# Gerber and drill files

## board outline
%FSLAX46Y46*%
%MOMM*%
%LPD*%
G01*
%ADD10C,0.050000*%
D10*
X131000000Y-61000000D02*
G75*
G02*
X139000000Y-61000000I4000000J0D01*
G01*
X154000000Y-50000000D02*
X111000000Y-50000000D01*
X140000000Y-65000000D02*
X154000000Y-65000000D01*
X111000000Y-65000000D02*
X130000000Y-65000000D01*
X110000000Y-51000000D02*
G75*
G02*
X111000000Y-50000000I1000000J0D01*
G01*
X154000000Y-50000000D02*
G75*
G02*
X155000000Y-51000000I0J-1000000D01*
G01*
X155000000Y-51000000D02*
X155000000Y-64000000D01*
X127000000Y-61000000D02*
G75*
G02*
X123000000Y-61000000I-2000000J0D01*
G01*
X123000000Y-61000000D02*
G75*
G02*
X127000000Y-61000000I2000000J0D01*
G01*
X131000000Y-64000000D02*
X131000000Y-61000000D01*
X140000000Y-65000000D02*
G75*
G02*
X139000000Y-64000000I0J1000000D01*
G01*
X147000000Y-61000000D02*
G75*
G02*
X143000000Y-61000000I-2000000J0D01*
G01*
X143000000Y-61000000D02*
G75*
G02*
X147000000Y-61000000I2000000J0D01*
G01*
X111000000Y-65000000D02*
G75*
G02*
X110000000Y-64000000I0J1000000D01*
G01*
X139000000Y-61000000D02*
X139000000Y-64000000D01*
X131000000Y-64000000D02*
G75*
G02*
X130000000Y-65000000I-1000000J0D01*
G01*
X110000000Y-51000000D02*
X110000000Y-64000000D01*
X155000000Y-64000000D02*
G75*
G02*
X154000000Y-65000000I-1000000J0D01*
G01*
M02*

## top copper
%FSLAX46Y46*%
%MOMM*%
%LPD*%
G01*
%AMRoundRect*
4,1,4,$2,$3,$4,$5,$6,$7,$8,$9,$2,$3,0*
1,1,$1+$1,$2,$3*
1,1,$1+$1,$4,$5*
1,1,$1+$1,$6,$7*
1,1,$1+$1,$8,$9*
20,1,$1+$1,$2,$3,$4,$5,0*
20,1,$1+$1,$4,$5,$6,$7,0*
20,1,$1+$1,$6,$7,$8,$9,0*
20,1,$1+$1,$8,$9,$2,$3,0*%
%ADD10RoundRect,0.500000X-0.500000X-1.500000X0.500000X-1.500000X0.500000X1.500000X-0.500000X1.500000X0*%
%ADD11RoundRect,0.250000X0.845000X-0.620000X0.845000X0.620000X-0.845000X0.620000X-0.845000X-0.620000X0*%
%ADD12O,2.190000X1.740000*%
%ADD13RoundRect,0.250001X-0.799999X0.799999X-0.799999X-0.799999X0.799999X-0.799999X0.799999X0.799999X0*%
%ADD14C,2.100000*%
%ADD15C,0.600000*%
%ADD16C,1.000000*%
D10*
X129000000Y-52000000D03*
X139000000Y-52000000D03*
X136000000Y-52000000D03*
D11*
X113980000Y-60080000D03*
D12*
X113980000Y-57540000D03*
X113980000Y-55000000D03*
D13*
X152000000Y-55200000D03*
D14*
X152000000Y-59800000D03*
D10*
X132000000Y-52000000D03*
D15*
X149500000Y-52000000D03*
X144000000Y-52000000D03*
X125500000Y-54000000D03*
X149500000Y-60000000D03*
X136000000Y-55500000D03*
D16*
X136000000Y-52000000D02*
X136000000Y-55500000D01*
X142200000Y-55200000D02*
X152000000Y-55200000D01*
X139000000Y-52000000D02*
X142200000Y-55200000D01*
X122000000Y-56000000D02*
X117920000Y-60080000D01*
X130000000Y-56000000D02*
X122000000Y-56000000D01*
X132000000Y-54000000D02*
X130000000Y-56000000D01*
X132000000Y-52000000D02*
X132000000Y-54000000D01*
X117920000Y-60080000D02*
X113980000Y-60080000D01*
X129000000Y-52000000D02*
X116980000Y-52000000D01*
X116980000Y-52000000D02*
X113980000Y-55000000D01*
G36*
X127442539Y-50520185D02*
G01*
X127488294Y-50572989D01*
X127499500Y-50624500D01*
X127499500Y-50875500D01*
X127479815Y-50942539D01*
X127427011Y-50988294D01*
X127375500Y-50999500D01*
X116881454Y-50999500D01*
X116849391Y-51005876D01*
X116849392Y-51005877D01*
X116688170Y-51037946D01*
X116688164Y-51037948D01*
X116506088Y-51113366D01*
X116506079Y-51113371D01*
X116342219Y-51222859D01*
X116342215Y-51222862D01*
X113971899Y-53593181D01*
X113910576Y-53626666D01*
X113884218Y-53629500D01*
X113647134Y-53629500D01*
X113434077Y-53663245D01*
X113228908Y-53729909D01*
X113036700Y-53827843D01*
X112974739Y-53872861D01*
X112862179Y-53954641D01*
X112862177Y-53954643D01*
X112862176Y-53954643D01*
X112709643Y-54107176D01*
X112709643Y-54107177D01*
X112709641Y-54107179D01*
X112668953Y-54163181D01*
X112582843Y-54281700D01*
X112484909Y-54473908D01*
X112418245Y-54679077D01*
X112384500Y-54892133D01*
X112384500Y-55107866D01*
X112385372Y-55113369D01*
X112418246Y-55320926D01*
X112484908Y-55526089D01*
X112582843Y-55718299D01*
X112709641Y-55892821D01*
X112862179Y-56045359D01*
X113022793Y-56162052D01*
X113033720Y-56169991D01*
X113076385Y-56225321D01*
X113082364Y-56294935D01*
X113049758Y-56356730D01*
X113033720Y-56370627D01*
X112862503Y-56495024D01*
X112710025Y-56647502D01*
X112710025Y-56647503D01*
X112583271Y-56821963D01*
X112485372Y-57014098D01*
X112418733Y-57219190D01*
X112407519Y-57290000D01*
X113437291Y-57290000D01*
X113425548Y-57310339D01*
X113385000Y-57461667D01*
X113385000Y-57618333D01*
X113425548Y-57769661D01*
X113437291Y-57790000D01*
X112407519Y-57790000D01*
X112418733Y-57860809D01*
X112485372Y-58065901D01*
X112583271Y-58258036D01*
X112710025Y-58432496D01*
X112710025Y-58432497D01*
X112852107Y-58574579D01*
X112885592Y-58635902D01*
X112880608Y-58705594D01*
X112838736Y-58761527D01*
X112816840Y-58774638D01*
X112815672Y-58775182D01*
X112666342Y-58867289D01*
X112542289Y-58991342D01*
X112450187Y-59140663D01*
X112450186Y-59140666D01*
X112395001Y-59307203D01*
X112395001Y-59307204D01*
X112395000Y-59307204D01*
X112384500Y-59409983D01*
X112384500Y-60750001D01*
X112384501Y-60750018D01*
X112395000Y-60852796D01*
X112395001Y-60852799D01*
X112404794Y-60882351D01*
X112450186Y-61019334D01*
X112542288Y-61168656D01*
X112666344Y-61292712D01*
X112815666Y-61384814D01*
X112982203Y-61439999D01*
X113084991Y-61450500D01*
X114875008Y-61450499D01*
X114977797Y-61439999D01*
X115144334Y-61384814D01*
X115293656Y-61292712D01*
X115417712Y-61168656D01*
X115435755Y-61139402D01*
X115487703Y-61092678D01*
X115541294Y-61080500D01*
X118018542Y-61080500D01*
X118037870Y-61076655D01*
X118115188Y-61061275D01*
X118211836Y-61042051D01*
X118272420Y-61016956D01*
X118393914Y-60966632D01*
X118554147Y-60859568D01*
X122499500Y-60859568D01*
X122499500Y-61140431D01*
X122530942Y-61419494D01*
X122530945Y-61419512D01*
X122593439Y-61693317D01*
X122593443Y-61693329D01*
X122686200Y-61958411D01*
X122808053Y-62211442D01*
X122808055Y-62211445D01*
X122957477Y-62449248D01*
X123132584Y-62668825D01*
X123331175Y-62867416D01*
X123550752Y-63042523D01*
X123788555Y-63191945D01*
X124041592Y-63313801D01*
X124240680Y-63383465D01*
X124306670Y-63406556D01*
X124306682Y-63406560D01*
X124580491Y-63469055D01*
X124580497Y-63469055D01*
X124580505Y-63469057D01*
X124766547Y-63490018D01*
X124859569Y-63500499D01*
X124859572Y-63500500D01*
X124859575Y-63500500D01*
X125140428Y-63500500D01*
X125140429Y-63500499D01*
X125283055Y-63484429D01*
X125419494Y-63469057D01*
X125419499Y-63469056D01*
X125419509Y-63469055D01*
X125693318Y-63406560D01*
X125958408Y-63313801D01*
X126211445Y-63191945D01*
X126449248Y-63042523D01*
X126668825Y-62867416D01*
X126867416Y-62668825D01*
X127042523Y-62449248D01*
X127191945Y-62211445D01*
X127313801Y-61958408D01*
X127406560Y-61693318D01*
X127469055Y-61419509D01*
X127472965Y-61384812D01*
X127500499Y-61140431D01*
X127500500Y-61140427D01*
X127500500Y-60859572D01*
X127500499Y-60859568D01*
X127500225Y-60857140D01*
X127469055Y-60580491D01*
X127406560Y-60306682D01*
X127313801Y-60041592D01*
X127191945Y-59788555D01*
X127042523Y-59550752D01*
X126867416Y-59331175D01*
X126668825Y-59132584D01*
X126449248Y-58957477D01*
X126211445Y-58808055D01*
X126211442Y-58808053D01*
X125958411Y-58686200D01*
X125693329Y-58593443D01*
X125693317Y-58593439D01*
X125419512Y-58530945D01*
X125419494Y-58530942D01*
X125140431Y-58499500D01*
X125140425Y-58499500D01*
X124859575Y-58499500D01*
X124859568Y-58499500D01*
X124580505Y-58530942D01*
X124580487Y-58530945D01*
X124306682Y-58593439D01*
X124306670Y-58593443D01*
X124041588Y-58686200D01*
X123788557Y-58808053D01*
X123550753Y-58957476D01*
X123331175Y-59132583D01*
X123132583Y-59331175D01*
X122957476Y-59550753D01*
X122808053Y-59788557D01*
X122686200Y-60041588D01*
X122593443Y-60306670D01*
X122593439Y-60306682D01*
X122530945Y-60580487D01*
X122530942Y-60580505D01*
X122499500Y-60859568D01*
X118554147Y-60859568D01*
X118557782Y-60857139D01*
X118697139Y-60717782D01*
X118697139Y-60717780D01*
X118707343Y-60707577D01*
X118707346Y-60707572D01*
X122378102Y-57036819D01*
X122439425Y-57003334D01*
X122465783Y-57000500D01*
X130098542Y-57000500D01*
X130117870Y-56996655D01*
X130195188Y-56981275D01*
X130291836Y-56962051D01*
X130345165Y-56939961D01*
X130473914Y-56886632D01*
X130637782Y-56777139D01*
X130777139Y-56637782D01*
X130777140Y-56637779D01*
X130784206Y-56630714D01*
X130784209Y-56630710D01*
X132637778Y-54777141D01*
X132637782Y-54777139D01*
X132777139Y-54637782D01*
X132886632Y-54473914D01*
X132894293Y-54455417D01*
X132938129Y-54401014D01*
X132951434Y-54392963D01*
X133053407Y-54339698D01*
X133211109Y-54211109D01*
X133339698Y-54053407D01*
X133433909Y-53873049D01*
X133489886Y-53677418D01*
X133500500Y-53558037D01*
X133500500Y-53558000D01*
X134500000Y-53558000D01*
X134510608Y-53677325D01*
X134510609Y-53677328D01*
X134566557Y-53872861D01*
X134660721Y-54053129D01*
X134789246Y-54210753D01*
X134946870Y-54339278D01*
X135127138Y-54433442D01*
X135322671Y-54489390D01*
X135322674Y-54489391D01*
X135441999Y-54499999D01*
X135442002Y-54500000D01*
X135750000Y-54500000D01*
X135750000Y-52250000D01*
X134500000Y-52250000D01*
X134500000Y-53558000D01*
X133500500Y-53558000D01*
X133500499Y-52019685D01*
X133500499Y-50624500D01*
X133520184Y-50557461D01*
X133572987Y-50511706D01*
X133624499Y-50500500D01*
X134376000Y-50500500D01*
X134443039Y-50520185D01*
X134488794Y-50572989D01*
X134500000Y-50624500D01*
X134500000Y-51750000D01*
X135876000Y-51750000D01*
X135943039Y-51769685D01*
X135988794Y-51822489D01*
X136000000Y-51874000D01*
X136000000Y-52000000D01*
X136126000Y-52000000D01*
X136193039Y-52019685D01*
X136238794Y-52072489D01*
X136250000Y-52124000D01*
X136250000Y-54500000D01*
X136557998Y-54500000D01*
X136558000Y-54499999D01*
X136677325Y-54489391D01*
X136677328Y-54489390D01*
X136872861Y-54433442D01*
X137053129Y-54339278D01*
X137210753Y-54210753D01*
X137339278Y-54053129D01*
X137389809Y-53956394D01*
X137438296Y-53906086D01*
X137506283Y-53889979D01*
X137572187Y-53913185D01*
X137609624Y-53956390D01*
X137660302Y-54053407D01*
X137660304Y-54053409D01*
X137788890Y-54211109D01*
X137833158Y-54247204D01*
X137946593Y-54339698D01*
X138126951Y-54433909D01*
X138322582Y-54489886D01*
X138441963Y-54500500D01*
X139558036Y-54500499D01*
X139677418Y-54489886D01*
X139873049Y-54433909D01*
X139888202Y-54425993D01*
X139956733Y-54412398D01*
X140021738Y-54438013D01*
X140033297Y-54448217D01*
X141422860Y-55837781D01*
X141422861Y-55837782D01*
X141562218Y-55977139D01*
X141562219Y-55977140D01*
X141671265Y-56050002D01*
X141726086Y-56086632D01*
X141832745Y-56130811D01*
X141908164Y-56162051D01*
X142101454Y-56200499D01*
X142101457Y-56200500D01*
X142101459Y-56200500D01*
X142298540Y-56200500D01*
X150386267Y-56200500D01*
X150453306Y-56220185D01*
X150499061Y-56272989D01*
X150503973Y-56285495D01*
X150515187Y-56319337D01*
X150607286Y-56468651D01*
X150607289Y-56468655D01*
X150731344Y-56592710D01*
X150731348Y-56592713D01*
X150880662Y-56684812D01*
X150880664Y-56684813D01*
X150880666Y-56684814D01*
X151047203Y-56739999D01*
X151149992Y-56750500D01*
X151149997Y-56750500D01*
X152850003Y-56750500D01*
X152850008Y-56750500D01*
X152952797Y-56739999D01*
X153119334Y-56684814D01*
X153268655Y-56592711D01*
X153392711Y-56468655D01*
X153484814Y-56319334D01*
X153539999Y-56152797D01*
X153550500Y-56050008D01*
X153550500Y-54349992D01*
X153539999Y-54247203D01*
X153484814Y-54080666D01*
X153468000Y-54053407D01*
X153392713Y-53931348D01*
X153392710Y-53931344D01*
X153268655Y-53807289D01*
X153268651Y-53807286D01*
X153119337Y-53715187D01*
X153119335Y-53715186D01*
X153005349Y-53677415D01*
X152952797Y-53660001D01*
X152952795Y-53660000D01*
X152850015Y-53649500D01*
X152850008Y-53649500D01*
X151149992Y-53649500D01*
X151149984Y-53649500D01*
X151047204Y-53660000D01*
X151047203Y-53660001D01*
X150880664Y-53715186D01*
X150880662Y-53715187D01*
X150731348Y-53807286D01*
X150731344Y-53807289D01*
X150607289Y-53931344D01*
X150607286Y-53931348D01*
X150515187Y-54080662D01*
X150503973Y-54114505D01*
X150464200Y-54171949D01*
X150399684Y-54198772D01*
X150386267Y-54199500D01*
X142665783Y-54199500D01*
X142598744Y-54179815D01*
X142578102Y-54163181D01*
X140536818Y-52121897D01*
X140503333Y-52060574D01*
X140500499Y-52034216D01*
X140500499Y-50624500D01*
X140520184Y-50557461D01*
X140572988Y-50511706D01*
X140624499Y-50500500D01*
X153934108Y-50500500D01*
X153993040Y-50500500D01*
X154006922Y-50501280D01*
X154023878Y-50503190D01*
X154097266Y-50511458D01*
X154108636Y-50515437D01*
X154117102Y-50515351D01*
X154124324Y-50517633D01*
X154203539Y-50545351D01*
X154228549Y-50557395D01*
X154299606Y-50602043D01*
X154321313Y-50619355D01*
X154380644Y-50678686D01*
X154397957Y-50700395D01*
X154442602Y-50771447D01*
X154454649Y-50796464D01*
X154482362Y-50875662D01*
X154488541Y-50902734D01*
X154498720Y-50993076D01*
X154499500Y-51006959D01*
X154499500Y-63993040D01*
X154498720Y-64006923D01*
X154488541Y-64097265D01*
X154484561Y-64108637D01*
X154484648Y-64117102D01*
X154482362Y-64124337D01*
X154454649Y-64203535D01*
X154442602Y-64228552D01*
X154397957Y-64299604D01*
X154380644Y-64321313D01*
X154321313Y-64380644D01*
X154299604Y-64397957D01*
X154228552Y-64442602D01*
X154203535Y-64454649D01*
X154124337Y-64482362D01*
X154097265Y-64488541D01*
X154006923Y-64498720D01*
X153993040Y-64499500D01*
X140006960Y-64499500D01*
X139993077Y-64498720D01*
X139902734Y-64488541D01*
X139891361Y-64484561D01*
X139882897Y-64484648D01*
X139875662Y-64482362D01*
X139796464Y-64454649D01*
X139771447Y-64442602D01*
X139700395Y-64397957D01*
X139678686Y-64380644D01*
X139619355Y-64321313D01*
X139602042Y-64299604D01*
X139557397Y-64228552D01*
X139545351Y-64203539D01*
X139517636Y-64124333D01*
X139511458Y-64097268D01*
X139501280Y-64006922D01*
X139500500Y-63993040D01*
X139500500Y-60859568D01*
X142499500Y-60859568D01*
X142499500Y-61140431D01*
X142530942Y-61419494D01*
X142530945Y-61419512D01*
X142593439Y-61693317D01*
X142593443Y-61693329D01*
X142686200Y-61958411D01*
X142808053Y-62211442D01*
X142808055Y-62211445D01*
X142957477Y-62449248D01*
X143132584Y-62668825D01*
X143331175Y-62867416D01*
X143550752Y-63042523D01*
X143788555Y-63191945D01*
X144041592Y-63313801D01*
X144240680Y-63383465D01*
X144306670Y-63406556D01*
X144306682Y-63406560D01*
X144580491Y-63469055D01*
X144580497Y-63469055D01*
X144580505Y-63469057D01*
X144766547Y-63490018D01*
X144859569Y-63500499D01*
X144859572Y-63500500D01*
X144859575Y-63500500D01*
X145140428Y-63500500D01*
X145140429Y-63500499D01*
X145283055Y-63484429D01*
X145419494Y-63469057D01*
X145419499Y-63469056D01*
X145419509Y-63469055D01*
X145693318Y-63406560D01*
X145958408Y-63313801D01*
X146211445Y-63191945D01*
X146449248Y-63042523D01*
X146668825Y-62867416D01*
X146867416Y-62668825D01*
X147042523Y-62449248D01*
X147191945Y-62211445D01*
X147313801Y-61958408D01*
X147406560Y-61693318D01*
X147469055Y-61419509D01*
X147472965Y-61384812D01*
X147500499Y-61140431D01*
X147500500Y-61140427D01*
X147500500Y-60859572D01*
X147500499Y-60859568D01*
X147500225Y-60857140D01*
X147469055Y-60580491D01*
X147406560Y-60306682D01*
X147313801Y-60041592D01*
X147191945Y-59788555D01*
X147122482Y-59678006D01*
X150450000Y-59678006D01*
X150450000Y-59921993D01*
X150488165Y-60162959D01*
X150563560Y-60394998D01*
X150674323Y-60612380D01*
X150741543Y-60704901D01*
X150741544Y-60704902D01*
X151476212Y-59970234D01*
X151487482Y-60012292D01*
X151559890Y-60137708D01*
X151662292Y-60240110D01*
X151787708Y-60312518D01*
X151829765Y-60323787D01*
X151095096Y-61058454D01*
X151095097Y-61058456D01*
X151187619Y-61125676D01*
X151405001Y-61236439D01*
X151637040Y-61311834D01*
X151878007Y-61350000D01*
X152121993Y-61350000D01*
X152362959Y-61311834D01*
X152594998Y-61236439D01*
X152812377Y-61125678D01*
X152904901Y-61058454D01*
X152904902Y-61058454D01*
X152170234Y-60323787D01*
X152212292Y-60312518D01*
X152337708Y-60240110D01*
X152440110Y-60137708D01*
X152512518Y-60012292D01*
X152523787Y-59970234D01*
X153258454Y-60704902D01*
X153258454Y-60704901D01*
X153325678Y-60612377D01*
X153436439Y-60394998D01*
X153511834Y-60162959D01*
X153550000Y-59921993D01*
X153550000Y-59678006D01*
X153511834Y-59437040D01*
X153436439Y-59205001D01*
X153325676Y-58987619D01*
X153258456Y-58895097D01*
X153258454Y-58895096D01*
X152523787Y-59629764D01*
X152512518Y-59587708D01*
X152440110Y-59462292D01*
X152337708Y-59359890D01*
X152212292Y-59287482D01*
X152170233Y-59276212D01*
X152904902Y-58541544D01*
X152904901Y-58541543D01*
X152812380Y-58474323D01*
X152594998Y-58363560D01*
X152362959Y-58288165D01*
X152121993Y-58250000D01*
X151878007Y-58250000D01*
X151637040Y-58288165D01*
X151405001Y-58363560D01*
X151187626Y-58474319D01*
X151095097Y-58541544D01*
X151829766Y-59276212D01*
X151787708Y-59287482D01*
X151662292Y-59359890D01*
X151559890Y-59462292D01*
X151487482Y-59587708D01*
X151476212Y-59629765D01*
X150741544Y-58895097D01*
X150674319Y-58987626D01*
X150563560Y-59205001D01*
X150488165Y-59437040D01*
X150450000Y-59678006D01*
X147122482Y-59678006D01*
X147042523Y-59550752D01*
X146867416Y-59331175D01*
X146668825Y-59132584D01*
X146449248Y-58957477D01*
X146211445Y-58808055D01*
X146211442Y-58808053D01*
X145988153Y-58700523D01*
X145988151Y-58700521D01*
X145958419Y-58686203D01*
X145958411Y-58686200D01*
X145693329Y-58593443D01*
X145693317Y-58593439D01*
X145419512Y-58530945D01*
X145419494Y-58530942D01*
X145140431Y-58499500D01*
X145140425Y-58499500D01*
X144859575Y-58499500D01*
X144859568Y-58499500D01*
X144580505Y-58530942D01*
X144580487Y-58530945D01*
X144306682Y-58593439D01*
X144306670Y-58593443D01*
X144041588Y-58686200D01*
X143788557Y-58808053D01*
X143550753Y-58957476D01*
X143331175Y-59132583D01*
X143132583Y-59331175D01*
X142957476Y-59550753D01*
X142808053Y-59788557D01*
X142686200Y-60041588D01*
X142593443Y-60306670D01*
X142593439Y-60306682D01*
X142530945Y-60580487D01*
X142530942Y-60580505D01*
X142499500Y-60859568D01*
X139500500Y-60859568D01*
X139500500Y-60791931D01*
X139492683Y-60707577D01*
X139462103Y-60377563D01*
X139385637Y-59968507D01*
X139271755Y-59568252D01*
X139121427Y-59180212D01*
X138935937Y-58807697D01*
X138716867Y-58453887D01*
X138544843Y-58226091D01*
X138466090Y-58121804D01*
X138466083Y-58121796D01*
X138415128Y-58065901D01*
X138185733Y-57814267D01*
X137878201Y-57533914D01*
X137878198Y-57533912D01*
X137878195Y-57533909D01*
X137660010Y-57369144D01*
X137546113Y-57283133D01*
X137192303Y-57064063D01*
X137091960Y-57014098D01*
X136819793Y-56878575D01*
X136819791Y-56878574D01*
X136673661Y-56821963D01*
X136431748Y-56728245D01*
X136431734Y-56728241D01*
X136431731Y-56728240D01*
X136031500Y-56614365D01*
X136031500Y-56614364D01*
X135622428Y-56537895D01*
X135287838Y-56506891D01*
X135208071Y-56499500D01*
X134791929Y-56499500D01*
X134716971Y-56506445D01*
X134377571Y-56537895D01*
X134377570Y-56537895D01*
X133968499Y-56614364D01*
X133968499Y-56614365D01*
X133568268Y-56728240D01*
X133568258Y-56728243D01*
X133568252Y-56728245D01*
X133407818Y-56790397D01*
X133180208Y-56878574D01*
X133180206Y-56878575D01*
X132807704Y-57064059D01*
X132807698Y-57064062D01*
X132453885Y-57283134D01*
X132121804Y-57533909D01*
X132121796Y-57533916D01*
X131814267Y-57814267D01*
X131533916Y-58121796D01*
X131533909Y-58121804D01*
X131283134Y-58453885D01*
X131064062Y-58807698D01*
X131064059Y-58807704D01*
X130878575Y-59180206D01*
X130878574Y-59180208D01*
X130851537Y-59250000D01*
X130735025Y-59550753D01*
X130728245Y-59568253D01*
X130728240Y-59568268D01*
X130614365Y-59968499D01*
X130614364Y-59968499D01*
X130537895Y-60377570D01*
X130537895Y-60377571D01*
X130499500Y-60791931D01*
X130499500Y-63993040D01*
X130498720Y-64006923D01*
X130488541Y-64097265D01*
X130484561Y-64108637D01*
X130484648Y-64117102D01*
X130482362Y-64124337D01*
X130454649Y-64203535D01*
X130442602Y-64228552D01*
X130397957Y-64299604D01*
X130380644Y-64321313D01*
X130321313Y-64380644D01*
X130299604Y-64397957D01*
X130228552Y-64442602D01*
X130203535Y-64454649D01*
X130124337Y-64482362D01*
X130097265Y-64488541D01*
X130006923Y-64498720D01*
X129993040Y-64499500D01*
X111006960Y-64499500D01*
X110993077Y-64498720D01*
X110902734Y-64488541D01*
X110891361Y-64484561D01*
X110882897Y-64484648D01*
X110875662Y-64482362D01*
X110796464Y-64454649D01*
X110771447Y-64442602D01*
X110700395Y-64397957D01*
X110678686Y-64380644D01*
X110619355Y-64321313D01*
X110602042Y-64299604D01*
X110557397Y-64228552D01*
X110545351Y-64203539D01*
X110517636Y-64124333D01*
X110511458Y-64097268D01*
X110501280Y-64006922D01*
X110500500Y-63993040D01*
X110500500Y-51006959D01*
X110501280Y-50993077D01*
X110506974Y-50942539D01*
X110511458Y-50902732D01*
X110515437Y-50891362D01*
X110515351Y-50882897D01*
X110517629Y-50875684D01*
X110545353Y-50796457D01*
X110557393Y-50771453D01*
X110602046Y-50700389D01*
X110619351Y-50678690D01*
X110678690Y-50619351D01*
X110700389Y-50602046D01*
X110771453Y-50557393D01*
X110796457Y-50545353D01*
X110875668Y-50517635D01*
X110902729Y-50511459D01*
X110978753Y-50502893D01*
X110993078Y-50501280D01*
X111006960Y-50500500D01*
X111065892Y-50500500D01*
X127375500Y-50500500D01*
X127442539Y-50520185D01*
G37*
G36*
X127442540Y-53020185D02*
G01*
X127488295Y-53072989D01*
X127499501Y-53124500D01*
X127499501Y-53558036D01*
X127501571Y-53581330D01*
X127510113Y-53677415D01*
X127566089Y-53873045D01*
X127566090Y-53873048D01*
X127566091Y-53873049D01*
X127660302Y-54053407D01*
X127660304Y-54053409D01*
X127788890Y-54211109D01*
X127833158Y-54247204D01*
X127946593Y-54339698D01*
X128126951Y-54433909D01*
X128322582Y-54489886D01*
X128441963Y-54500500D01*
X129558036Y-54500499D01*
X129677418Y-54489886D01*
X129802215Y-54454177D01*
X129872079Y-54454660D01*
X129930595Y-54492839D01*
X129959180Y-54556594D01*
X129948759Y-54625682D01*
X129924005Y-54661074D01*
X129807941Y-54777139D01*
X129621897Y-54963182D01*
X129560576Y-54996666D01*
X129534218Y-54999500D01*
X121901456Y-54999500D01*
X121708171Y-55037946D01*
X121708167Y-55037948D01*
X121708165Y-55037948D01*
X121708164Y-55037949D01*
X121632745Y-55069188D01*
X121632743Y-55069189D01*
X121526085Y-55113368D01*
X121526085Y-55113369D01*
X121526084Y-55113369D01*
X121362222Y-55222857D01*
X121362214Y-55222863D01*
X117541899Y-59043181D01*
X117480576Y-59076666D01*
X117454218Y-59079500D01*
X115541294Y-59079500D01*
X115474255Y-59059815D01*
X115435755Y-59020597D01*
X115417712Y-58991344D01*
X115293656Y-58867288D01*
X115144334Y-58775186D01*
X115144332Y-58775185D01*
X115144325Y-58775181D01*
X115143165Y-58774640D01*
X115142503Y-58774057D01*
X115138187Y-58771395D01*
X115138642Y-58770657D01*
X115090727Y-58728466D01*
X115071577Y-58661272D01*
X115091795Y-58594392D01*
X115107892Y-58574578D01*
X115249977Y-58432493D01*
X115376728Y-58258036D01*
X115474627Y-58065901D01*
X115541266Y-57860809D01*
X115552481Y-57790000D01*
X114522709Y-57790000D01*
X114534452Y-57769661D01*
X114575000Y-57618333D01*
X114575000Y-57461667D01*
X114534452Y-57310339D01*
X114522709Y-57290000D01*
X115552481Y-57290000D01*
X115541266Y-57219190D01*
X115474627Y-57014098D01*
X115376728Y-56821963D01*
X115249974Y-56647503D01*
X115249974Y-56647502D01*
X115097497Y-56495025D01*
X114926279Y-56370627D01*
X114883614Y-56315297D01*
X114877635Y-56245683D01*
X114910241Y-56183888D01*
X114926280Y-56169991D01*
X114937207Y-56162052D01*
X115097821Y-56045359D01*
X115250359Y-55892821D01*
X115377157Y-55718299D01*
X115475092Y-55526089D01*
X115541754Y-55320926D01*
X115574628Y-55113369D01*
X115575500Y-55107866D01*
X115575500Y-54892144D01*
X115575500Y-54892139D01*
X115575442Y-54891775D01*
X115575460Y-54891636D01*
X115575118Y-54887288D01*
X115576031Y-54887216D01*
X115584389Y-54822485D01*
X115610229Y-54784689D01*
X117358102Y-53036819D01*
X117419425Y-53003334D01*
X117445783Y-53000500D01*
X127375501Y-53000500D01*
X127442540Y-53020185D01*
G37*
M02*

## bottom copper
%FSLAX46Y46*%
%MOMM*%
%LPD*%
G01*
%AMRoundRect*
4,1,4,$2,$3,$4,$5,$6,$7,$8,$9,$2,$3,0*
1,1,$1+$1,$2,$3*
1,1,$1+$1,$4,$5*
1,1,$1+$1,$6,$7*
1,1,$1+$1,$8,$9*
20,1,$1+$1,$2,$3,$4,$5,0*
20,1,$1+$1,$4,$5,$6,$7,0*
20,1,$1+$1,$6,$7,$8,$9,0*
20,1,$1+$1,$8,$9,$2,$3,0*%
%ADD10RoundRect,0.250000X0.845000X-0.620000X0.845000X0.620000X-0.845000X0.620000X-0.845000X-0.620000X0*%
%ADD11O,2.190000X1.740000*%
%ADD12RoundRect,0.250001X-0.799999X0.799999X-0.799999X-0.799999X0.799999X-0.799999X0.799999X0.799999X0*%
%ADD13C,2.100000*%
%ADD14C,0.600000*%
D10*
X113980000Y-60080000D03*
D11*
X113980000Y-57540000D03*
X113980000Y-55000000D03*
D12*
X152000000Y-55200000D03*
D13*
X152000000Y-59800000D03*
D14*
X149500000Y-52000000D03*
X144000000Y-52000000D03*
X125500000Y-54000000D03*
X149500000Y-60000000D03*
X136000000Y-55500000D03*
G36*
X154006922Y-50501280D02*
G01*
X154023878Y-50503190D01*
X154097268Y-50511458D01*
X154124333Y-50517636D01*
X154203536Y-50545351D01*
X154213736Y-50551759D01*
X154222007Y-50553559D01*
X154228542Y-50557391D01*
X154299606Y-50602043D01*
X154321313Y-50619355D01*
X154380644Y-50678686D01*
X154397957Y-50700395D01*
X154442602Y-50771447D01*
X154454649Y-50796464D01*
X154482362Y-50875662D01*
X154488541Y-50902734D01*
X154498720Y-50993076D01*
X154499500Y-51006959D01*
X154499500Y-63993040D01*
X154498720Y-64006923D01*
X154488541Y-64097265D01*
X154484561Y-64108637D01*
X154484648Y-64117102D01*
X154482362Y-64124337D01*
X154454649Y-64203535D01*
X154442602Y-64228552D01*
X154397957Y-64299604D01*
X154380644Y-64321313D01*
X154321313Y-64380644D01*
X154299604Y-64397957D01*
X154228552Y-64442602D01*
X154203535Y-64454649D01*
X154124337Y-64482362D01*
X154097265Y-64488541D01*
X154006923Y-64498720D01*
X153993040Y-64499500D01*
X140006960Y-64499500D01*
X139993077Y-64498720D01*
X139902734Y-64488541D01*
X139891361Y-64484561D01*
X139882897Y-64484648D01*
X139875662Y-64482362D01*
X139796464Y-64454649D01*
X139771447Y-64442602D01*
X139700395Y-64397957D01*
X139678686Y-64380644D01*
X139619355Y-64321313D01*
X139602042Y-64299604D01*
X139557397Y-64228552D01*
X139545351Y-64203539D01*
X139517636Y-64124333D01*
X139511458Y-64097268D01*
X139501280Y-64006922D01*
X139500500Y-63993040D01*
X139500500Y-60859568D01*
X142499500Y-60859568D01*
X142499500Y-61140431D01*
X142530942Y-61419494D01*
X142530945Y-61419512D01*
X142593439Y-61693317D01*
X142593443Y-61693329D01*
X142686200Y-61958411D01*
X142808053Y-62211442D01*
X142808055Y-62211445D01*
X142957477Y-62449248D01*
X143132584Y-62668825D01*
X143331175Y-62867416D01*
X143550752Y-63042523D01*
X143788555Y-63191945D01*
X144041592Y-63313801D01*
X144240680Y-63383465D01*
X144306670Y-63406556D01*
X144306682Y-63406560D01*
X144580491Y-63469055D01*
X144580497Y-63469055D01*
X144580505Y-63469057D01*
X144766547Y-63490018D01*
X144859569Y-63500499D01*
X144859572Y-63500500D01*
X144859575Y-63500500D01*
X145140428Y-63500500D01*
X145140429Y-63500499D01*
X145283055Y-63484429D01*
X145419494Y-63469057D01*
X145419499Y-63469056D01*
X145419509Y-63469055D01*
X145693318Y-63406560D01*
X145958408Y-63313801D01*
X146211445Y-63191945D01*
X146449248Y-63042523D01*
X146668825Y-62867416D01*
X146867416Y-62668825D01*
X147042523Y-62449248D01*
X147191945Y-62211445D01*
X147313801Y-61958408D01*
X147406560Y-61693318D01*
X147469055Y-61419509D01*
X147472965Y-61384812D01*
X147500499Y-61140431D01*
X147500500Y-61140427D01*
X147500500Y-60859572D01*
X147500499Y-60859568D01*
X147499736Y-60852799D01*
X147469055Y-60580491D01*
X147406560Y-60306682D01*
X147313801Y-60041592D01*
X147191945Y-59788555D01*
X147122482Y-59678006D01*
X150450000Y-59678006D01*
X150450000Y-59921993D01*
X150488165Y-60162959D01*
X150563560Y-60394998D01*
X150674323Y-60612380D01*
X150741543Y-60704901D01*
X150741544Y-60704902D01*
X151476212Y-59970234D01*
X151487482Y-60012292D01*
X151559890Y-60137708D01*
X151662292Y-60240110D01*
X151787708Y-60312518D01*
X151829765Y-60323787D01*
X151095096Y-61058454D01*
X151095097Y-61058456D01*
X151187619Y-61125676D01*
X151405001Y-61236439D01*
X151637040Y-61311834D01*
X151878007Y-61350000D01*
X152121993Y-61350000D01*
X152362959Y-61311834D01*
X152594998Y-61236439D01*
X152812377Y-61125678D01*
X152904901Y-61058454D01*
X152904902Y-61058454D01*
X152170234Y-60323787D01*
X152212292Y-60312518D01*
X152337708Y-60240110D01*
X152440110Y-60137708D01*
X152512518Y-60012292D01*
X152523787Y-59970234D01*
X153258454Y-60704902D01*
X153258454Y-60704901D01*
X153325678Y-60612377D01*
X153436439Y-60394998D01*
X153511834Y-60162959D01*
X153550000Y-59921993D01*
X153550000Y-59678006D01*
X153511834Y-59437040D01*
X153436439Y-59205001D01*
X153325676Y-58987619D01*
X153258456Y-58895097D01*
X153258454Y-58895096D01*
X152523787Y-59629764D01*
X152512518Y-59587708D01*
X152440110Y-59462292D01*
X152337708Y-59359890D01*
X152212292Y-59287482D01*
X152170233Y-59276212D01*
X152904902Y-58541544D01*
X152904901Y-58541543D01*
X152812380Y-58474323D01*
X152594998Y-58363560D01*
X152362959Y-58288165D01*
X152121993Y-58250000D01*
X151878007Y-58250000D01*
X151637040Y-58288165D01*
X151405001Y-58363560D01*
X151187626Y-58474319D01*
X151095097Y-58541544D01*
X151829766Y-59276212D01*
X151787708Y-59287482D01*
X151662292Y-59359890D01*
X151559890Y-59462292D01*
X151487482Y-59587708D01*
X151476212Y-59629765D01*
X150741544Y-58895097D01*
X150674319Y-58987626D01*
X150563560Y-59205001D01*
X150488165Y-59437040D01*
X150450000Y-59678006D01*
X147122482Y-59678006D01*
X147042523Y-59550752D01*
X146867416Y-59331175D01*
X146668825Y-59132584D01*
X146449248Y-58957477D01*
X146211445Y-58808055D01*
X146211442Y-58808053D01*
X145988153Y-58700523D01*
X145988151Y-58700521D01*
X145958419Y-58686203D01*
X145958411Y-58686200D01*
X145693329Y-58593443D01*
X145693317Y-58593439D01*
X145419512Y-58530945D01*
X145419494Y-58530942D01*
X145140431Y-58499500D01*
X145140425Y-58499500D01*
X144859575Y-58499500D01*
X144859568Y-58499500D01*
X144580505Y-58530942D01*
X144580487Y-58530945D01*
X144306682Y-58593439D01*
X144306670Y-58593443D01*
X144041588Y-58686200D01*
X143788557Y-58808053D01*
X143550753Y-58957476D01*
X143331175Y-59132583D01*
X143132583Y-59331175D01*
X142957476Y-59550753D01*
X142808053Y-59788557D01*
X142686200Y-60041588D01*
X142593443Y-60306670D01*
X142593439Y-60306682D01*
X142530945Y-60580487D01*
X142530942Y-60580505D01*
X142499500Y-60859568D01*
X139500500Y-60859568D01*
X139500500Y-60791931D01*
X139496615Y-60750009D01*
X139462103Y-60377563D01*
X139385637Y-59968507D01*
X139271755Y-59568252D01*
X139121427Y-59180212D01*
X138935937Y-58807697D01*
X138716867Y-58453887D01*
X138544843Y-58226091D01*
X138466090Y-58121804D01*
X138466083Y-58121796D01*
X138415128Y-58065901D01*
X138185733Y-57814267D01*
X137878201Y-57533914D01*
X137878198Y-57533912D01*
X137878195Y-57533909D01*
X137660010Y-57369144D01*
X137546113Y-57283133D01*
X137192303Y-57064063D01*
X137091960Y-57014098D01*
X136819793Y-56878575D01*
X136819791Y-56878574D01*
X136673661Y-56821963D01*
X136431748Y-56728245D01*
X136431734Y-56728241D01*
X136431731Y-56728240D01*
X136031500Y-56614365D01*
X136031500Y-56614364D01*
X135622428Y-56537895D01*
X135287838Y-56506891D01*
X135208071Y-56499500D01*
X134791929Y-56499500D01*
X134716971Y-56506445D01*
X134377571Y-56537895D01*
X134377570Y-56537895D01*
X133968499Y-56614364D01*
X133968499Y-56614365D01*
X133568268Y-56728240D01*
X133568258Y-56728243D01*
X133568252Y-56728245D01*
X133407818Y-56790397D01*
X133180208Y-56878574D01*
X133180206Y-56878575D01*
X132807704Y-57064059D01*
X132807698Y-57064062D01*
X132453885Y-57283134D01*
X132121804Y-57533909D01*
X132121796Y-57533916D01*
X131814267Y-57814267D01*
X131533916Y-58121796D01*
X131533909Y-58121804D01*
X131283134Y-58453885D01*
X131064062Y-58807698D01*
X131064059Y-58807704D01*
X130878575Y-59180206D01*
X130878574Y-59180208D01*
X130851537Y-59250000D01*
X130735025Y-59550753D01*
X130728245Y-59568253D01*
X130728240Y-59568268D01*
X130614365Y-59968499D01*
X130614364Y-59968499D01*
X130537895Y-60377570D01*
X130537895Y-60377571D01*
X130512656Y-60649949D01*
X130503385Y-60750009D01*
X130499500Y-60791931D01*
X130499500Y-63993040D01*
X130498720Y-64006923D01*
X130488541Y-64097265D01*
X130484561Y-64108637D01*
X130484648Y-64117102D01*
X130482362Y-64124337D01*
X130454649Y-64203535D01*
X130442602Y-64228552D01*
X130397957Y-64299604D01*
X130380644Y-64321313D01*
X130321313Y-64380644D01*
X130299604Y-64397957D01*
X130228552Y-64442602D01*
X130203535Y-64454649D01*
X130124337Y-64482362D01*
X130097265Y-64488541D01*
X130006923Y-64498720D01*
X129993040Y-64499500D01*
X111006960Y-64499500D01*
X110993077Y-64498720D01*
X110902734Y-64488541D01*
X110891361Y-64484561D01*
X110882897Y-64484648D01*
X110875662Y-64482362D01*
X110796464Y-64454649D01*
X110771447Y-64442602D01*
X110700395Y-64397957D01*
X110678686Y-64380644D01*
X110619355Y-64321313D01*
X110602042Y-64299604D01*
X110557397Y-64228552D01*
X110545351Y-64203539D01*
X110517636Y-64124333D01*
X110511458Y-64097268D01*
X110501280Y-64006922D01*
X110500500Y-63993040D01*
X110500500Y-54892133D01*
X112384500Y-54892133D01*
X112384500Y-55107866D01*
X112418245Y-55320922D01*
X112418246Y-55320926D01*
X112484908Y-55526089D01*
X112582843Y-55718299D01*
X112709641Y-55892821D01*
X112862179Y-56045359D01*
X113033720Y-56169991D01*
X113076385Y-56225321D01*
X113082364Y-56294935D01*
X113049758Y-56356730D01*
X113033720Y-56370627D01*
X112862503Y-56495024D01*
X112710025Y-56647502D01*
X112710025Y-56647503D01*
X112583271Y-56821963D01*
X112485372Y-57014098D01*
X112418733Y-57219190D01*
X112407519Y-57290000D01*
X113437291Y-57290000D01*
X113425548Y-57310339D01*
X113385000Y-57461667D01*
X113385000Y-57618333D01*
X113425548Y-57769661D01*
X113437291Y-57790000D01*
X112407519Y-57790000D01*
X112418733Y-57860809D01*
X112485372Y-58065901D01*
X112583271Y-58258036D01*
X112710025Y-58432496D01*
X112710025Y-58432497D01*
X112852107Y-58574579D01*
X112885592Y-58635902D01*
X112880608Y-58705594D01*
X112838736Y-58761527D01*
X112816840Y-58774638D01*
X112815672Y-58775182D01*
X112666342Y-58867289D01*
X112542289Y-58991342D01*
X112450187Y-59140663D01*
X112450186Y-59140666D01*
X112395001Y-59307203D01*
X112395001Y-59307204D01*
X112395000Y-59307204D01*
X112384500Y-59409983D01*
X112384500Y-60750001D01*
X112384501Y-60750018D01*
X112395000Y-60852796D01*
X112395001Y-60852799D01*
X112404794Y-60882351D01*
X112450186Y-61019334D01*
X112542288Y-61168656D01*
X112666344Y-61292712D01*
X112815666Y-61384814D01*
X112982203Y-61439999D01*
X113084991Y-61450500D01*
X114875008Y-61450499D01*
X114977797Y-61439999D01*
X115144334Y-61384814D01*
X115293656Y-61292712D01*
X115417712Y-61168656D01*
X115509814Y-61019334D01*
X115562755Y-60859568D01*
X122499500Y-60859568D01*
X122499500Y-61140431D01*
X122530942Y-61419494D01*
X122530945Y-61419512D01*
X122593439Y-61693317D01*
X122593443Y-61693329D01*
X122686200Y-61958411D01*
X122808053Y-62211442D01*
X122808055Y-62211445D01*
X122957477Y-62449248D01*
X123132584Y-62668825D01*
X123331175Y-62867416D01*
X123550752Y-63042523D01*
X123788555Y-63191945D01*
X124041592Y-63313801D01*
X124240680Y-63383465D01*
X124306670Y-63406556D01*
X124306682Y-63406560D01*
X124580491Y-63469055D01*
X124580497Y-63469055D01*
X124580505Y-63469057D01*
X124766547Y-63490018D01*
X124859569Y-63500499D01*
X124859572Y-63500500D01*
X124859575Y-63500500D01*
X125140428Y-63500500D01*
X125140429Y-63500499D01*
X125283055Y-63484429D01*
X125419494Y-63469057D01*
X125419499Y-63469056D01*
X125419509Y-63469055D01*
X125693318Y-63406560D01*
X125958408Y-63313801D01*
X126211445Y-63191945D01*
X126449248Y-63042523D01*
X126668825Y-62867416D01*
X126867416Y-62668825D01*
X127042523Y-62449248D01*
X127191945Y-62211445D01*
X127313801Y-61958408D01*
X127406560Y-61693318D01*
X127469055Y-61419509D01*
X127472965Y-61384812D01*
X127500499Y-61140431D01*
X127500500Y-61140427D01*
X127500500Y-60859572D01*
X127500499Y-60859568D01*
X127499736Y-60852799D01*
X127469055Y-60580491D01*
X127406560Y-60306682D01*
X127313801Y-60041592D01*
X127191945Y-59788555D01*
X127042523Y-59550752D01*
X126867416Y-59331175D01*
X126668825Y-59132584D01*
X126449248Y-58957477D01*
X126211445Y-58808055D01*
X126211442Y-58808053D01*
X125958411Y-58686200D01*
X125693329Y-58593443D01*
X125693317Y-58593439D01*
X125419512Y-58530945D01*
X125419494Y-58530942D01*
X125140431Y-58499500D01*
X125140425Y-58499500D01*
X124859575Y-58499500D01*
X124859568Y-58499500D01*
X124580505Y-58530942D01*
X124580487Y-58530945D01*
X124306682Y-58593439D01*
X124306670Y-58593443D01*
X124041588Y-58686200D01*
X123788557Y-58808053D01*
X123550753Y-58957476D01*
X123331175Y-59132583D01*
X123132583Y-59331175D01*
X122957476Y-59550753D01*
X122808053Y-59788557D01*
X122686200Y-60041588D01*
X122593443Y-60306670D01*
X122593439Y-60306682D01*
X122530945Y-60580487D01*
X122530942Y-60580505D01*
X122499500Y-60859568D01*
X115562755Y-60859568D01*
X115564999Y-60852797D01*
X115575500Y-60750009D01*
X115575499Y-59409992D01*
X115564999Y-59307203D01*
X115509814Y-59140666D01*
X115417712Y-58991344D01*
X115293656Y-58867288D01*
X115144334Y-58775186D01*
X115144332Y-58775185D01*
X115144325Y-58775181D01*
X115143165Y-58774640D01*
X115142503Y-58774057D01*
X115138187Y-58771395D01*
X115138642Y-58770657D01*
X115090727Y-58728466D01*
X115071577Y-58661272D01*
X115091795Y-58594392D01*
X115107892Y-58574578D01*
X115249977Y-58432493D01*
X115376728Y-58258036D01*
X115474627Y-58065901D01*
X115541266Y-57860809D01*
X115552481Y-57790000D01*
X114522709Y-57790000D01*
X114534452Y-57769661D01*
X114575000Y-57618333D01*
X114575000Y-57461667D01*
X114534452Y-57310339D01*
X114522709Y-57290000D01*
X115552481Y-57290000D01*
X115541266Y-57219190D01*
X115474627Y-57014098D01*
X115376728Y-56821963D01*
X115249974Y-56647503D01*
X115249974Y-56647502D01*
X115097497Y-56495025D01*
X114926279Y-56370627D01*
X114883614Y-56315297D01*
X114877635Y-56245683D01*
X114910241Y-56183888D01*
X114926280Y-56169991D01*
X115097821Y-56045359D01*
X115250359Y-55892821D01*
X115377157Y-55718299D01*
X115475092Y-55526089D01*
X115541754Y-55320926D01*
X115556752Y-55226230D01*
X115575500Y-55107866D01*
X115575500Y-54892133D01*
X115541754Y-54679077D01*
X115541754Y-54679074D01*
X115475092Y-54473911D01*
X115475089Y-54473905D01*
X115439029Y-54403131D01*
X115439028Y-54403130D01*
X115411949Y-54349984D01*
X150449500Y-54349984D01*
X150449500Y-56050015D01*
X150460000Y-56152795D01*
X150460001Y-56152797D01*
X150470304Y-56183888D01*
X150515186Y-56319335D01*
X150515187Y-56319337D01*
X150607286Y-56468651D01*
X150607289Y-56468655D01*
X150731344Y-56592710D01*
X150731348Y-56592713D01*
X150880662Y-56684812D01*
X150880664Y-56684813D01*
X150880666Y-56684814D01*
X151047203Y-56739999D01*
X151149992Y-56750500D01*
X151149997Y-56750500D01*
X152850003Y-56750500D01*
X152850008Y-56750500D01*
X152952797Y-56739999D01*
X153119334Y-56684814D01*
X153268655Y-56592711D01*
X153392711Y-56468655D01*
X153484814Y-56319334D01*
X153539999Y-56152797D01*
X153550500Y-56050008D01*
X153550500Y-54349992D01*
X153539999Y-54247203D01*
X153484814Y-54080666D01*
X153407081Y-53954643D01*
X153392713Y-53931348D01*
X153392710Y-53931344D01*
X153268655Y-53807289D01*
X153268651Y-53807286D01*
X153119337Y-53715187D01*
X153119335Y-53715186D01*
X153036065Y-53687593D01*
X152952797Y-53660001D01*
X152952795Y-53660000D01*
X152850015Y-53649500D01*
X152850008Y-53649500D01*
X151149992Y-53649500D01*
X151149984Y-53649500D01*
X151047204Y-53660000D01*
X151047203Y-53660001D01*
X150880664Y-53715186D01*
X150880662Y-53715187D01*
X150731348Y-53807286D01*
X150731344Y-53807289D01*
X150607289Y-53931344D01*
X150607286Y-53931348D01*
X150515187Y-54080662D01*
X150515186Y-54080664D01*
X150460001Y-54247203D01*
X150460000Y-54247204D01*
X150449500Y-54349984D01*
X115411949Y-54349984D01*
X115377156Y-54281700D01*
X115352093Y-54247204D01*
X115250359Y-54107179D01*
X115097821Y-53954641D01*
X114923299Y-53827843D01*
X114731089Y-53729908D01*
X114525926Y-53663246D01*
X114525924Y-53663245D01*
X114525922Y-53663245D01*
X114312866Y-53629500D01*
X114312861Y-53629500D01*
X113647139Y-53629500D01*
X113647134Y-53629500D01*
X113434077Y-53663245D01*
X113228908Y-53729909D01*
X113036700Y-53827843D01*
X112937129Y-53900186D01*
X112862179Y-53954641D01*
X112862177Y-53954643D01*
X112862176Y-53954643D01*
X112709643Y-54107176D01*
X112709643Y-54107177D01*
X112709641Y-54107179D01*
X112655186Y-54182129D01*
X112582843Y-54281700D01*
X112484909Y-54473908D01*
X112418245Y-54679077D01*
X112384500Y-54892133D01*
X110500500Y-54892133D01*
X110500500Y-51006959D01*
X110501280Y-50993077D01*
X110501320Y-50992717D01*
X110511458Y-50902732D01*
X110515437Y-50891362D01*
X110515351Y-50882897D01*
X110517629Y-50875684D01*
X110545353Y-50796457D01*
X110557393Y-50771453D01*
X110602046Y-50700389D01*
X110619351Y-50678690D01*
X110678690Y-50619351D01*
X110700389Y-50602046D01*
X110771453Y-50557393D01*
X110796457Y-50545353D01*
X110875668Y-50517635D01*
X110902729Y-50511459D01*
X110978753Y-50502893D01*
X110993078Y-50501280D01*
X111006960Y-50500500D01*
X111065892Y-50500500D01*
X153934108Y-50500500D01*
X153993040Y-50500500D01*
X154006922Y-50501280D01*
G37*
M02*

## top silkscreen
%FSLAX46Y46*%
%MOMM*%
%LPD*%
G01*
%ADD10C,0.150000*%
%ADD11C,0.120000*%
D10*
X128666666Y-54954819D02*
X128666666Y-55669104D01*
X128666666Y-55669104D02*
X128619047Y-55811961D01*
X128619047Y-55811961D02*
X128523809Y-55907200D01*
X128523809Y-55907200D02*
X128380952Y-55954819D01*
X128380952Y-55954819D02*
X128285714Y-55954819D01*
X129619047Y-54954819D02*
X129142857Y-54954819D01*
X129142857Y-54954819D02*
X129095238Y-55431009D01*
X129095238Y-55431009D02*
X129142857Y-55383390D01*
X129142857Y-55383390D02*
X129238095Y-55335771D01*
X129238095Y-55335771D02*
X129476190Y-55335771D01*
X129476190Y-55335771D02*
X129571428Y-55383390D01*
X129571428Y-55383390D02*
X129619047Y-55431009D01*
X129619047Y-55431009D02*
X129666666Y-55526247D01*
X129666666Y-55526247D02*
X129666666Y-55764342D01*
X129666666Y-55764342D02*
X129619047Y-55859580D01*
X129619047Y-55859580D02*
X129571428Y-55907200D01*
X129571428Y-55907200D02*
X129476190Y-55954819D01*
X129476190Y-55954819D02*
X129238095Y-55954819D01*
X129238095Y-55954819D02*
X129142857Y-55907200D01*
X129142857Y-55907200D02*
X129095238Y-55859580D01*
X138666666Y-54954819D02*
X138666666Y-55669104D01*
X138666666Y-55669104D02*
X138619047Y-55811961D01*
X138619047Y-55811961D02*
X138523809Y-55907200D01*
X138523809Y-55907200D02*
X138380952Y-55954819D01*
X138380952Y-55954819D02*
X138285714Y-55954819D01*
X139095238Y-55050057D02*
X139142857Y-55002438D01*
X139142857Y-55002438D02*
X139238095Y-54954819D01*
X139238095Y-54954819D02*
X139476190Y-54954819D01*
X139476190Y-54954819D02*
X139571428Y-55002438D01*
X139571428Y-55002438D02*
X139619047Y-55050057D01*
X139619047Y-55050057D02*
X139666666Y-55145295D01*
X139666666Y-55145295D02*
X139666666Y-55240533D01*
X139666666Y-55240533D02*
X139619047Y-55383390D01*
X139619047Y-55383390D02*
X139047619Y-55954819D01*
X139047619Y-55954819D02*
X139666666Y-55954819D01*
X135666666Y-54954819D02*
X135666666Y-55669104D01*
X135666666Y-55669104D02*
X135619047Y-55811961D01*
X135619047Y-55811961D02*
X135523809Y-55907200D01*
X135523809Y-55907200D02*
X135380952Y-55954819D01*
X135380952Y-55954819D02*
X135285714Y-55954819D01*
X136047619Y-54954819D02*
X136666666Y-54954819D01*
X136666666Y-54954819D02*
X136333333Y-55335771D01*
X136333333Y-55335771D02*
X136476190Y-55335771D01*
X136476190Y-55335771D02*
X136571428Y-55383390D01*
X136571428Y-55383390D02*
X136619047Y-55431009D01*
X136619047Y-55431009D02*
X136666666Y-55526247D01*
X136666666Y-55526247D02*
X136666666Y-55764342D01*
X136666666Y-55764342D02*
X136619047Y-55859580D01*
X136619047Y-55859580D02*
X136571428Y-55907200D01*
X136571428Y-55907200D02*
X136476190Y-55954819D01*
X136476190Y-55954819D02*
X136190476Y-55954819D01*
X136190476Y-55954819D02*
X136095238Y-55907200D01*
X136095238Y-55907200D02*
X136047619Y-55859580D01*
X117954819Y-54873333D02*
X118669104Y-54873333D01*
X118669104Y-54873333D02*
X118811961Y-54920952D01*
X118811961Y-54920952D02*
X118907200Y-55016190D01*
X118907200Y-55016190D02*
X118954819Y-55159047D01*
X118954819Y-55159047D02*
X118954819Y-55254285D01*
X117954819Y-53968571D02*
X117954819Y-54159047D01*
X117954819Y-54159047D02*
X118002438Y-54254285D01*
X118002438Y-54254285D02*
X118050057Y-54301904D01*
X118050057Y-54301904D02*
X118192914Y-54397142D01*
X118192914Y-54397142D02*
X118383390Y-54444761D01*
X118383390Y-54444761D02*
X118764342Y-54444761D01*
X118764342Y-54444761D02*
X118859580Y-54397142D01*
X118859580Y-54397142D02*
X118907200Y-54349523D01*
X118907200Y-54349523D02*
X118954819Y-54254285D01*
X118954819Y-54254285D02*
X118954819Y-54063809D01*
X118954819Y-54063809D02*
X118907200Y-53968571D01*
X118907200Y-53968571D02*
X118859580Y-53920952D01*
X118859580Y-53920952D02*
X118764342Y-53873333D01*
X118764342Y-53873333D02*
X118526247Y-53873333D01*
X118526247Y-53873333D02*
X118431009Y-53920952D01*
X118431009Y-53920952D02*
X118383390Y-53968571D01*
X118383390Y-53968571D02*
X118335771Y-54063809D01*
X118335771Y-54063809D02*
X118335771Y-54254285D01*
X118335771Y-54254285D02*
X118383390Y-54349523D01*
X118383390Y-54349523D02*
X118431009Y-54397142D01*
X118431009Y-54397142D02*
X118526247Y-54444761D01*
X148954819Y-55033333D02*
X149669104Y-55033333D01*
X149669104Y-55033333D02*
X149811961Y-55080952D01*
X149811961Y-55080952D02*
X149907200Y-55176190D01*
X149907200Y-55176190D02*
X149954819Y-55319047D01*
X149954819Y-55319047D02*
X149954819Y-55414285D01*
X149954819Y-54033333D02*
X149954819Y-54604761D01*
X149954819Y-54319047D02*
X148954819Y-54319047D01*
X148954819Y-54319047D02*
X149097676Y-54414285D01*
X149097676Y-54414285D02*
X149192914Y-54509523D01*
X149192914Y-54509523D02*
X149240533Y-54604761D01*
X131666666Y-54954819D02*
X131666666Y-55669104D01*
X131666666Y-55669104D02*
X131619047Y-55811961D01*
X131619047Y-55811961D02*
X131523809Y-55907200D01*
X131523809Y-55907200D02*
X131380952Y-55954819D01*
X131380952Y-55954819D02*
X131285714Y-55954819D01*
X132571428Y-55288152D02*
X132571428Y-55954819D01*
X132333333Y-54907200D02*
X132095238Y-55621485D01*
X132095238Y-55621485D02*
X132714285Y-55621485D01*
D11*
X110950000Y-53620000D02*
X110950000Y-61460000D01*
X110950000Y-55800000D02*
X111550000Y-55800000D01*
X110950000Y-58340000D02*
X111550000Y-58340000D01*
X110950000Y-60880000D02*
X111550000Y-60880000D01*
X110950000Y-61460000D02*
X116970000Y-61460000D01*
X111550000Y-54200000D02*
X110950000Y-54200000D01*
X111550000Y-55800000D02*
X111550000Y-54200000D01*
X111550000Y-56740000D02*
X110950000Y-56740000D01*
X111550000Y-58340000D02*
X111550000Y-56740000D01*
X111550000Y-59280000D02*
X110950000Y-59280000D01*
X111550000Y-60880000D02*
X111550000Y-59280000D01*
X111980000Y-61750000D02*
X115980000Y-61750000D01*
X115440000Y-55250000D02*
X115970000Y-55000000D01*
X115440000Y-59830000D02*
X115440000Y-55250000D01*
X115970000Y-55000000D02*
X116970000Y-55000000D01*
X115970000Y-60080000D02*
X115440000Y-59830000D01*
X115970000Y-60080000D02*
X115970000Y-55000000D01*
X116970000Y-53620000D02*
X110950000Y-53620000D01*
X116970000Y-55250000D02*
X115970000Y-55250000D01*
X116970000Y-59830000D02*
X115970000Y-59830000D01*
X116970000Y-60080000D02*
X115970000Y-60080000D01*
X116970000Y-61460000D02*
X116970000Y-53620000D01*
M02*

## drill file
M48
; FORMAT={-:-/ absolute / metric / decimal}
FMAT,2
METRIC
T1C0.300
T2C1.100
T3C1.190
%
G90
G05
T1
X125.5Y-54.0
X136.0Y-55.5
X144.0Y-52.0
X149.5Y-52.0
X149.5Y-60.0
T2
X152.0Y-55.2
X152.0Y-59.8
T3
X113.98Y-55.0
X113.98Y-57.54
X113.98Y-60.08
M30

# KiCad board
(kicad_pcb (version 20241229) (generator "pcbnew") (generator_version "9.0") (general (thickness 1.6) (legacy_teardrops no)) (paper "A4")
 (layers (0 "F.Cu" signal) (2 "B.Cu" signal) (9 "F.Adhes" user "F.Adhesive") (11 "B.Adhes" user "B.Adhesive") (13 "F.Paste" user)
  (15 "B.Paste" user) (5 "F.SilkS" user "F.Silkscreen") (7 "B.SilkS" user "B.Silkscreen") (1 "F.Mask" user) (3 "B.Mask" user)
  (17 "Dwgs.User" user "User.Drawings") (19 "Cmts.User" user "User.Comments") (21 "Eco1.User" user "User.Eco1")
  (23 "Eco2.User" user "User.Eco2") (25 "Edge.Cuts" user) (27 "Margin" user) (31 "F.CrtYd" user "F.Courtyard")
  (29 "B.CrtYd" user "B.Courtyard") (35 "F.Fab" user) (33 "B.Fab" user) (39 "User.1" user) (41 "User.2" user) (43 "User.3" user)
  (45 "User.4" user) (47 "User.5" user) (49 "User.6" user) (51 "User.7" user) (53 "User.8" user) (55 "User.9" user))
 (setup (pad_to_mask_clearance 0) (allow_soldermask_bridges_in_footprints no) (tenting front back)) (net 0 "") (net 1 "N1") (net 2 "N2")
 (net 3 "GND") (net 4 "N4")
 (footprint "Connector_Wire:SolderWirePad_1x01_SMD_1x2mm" (layer "F.Cu") (at 129 52)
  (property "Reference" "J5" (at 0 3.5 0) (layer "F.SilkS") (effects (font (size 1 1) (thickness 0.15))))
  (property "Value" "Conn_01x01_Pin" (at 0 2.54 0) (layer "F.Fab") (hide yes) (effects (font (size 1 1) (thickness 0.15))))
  (pad "1" smd roundrect (at 0 0) (size 2 4) (layers "F.Cu" "F.Mask" "F.Paste") (roundrect_rratio 0.25) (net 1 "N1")))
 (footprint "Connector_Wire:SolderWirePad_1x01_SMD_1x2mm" (layer "F.Cu") (at 139 52)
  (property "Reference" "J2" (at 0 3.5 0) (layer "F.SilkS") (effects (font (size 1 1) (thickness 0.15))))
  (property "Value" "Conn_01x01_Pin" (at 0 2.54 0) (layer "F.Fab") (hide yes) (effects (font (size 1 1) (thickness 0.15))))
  (pad "1" smd roundrect (at 0 0) (size 2 4) (layers "F.Cu" "F.Mask" "F.Paste") (roundrect_rratio 0.25) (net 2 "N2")))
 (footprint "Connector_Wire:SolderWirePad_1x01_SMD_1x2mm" (layer "F.Cu") (at 136 52)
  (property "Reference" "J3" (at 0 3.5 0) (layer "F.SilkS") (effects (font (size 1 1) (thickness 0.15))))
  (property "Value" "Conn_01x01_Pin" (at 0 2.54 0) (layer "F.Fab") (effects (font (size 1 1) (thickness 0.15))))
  (pad "1" smd roundrect (at 0 0) (size 2 4) (layers "F.Cu" "F.Mask" "F.Paste") (roundrect_rratio 0.25) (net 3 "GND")))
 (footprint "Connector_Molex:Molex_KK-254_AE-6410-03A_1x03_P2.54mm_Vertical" (layer "F.Cu") (at 113.98 60.08 90)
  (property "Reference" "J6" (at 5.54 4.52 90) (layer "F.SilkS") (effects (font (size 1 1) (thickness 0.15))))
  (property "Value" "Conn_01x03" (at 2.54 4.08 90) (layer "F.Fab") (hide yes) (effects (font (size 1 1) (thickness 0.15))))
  (fp_line (start 6.46 -3.03) (end -1.38 -3.03) (stroke (width 0.12) (type solid)) (layer "F.SilkS"))
  (fp_line (start 4.28 -3.03) (end 4.28 -2.43) (stroke (width 0.12) (type solid)) (layer "F.SilkS"))
  (fp_line (start 1.74 -3.03) (end 1.74 -2.43) (stroke (width 0.12) (type solid)) (layer "F.SilkS"))
  (fp_line (start -0.8 -3.03) (end -0.8 -2.43) (stroke (width 0.12) (type solid)) (layer "F.SilkS"))
  (fp_line (start -1.38 -3.03) (end -1.38 2.99) (stroke (width 0.12) (type solid)) (layer "F.SilkS"))
  (fp_line (start 5.88 -2.43) (end 5.88 -3.03) (stroke (width 0.12) (type solid)) (layer "F.SilkS"))
  (fp_line (start 4.28 -2.43) (end 5.88 -2.43) (stroke (width 0.12) (type solid)) (layer "F.SilkS"))
  (fp_line (start 3.34 -2.43) (end 3.34 -3.03) (stroke (width 0.12) (type solid)) (layer "F.SilkS"))
  (fp_line (start 1.74 -2.43) (end 3.34 -2.43) (stroke (width 0.12) (type solid)) (layer "F.SilkS"))
  (fp_line (start 0.8 -2.43) (end 0.8 -3.03) (stroke (width 0.12) (type solid)) (layer "F.SilkS"))
  (fp_line (start -0.8 -2.43) (end 0.8 -2.43) (stroke (width 0.12) (type solid)) (layer "F.SilkS"))
  (fp_line (start -1.67 -2) (end -1.67 2) (stroke (width 0.12) (type solid)) (layer "F.SilkS"))
  (fp_line (start 4.83 1.46) (end 5.08 1.99) (stroke (width 0.12) (type solid)) (layer "F.SilkS"))
  (fp_line (start 0.25 1.46) (end 4.83 1.46) (stroke (width 0.12) (type solid)) (layer "F.SilkS"))
  (fp_line (start 5.08 1.99) (end 5.08 2.99) (stroke (width 0.12) (type solid)) (layer "F.SilkS"))
  (fp_line (start 0 1.99) (end 0.25 1.46) (stroke (width 0.12) (type solid)) (layer "F.SilkS"))
  (fp_line (start 0 1.99) (end 5.08 1.99) (stroke (width 0.12) (type solid)) (layer "F.SilkS"))
  (fp_line (start 6.46 2.99) (end 6.46 -3.03) (stroke (width 0.12) (type solid)) (layer "F.SilkS"))
  (fp_line (start 4.83 2.99) (end 4.83 1.99) (stroke (width 0.12) (type solid)) (layer "F.SilkS"))
  (fp_line (start 0.25 2.99) (end 0.25 1.99) (stroke (width 0.12) (type solid)) (layer "F.SilkS"))
  (fp_line (start 0 2.99) (end 0 1.99) (stroke (width 0.12) (type solid)) (layer "F.SilkS"))
  (fp_line (start -1.38 2.99) (end 6.46 2.99) (stroke (width 0.12) (type solid)) (layer "F.SilkS"))
  (pad "1" thru_hole roundrect (at 0 0 90) (size 1.74 2.19) (drill 1.19) (layers "*.Cu" "*.Mask") (remove_unused_layers no)
   (roundrect_rratio 0.143678) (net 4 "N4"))
  (pad "2" thru_hole oval (at 2.54 0 90) (size 1.74 2.19) (drill 1.19) (layers "*.Cu" "*.Mask") (remove_unused_layers no) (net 3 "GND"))
  (pad "3" thru_hole oval (at 5.08 0 90) (size 1.74 2.19) (drill 1.19) (layers "*.Cu" "*.Mask") (remove_unused_layers no) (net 1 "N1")))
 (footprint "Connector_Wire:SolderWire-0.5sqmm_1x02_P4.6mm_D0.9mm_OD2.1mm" (layer "F.Cu") (at 152 55.2 -90)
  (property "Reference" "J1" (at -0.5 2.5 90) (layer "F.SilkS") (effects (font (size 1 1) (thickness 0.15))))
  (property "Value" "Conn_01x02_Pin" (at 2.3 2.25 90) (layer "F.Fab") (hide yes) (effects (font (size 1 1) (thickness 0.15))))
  (pad "1" thru_hole roundrect (at 0 0 270) (size 2.1 2.1) (drill 1.1) (layers "*.Cu" "*.Mask") (remove_unused_layers no)
   (roundrect_rratio 0.119048) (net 2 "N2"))
  (pad "2" thru_hole circle (at 4.6 0 270) (size 2.1 2.1) (drill 1.1) (layers "*.Cu" "*.Mask") (remove_unused_layers no) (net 3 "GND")))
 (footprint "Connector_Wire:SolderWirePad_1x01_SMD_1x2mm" (layer "F.Cu") (at 132 52)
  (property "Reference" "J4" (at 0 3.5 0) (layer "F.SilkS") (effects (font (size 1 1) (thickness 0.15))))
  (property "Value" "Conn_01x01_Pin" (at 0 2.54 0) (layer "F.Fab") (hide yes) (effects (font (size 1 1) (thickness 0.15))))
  (pad "1" smd roundrect (at 0 0) (size 2 4) (layers "F.Cu" "F.Mask" "F.Paste") (roundrect_rratio 0.25) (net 4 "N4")))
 (gr_arc (start 131 61) (mid 135 57) (end 139 61) (stroke (width 0.05) (type default)) (layer "Edge.Cuts"))
 (gr_line (start 154 50) (end 111 50) (stroke (width 0.05) (type default)) (layer "Edge.Cuts"))
 (gr_line (start 140 65) (end 154 65) (stroke (width 0.05) (type default)) (layer "Edge.Cuts"))
 (gr_line (start 111 65) (end 130 65) (stroke (width 0.05) (type default)) (layer "Edge.Cuts"))
 (gr_arc (start 110 51) (mid 110.292893 50.292893) (end 111 50) (stroke (width 0.05) (type default)) (layer "Edge.Cuts"))
 (gr_arc (start 154 50) (mid 154.707107 50.292893) (end 155 51) (stroke (width 0.05) (type default)) (layer "Edge.Cuts"))
 (gr_line (start 155 51) (end 155 64) (stroke (width 0.05) (type default)) (layer "Edge.Cuts"))
 (gr_circle (center 125 61) (end 125 63) (stroke (width 0.05) (type default)) (fill no) (layer "Edge.Cuts"))
 (gr_line (start 131 64) (end 131 61) (stroke (width 0.05) (type default)) (layer "Edge.Cuts"))
 (gr_arc (start 140 65) (mid 139.292893 64.707107) (end 139 64) (stroke (width 0.05) (type default)) (layer "Edge.Cuts"))
 (gr_circle (center 145 61) (end 145 63) (stroke (width 0.05) (type default)) (fill no) (layer "Edge.Cuts"))
 (gr_arc (start 111 65) (mid 110.292893 64.707107) (end 110 64) (stroke (width 0.05) (type default)) (layer "Edge.Cuts"))
 (gr_line (start 139 61) (end 139 64) (stroke (width 0.05) (type default)) (layer "Edge.Cuts"))
 (gr_arc (start 131 64) (mid 130.707107 64.707107) (end 130 65) (stroke (width 0.05) (type default)) (layer "Edge.Cuts"))
 (gr_line (start 110 51) (end 110 64) (stroke (width 0.05) (type default)) (layer "Edge.Cuts"))
 (gr_arc (start 155 64) (mid 154.707107 64.707107) (end 154 65) (stroke (width 0.05) (type default)) (layer "Edge.Cuts"))
 (segment (start 136 52) (end 136 55.5) (width 1) (layer "F.Cu") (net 3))
 (via (at 149.5 52) (size 0.6) (drill 0.3) (layers "F.Cu" "B.Cu") (free yes) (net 3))
 (via (at 144 52) (size 0.6) (drill 0.3) (layers "F.Cu" "B.Cu") (free yes) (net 3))
 (via (at 125.5 54) (size 0.6) (drill 0.3) (layers "F.Cu" "B.Cu") (free yes) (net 3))
 (via (at 149.5 60) (size 0.6) (drill 0.3) (layers "F.Cu" "B.Cu") (free yes) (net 3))
 (via (at 136 55.5) (size 0.6) (drill 0.3) (layers "F.Cu" "B.Cu") (free yes) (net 3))
 (segment (start 142.2 55.2) (end 152 55.2) (width 1) (layer "F.Cu") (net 2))
 (segment (start 139 52) (end 142.2 55.2) (width 1) (layer "F.Cu") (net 2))
 (segment (start 122 56) (end 117.92 60.08) (width 1) (layer "F.Cu") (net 4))
 (segment (start 130 56) (end 122 56) (width 1) (layer "F.Cu") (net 4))
 (segment (start 132 54) (end 130 56) (width 1) (layer "F.Cu") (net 4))
 (segment (start 132 52) (end 132 54) (width 1) (layer "F.Cu") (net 4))
 (segment (start 117.92 60.08) (end 113.98 60.08) (width 1) (layer "F.Cu") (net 4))
 (segment (start 129 52) (end 116.98 52) (width 1) (layer "F.Cu") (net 1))
 (segment (start 116.98 52) (end 113.98 55) (width 1) (layer "F.Cu") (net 1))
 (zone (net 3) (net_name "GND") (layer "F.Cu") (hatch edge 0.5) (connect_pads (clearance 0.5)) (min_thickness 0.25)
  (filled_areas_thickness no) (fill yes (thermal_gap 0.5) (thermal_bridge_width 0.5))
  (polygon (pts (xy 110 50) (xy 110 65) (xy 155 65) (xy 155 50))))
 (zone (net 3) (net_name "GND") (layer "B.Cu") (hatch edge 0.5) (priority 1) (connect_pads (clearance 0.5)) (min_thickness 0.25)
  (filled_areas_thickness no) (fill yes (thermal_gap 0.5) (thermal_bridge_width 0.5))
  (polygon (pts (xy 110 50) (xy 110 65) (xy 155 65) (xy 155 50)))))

